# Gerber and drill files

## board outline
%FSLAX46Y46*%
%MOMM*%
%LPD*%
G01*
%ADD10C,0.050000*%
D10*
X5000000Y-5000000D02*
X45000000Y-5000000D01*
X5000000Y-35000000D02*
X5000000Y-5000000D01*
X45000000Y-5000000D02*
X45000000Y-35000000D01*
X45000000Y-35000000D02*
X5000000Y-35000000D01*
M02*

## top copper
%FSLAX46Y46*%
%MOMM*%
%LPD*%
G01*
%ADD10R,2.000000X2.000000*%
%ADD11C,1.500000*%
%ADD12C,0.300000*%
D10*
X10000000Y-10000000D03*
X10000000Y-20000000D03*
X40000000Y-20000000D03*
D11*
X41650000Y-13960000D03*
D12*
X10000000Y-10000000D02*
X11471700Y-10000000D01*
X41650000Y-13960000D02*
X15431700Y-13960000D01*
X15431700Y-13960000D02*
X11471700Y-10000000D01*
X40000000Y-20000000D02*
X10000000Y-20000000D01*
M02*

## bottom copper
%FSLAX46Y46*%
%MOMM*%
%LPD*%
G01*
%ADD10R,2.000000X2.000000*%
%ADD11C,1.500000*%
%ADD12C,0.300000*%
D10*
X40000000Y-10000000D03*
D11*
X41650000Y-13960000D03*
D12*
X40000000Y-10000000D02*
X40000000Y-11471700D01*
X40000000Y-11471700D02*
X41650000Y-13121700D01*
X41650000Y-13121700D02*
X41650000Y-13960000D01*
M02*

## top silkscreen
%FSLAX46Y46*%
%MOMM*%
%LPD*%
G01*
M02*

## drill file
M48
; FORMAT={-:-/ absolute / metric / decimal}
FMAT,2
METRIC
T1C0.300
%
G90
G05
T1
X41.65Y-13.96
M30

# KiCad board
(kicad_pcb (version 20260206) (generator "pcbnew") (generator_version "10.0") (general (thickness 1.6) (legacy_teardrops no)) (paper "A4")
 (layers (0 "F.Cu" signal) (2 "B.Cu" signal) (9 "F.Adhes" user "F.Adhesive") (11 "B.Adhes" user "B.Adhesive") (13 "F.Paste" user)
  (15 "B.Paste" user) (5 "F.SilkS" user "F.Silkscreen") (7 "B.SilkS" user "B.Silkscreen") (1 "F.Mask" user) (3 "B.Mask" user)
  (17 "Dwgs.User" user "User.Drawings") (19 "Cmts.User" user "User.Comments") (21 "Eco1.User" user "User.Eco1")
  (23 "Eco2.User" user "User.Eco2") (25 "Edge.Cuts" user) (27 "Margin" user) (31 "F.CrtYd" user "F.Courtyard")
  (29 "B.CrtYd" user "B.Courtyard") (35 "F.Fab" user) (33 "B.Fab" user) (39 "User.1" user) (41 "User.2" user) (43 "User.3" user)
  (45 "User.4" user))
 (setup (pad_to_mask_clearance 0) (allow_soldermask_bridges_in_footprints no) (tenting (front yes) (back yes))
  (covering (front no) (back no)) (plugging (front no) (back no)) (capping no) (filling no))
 (gr_line (start 5 5) (end 45 5) (stroke (width 0.05) (type default)) (layer "Edge.Cuts"))
 (gr_line (start 5 35) (end 5 5) (stroke (width 0.05) (type default)) (layer "Edge.Cuts"))
 (gr_line (start 45 5) (end 45 35) (stroke (width 0.05) (type default)) (layer "Edge.Cuts"))
 (gr_line (start 45 35) (end 5 35) (stroke (width 0.05) (type default)) (layer "Edge.Cuts"))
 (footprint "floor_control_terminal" (layer "F.Cu") (at 10 10)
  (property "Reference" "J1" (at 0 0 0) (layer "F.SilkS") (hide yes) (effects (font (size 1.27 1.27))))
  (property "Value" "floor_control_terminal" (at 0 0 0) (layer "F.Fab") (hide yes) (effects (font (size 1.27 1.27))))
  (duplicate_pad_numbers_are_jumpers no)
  (pad "1" smd rect (at 0 0) (size 2 2) (layers "F.Cu" "F.Paste" "F.Mask") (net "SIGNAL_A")))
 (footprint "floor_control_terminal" (layer "B.Cu") (at 40 10)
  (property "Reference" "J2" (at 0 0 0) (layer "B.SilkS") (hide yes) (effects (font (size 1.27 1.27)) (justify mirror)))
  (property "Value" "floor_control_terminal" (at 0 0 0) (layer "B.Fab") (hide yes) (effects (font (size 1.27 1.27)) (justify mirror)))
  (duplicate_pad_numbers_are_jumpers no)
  (pad "1" smd rect (at 0 0) (size 2 2) (layers "B.Cu" "B.Paste" "B.Mask") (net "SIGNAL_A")))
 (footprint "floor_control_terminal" (layer "F.Cu") (at 10 20)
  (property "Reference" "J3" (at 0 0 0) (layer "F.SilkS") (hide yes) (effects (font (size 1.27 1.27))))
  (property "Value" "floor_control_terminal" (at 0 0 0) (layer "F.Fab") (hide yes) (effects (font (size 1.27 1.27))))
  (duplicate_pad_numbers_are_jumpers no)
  (pad "1" smd rect (at 0 0) (size 2 2) (layers "F.Cu" "F.Paste" "F.Mask") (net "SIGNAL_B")))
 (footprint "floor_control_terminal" (layer "F.Cu") (at 40 20)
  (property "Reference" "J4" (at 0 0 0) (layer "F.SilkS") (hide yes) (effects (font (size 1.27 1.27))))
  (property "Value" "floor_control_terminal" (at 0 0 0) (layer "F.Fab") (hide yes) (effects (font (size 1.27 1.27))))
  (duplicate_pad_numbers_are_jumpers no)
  (pad "1" smd rect (at 0 0) (size 2 2) (layers "F.Cu" "F.Paste" "F.Mask") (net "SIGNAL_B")))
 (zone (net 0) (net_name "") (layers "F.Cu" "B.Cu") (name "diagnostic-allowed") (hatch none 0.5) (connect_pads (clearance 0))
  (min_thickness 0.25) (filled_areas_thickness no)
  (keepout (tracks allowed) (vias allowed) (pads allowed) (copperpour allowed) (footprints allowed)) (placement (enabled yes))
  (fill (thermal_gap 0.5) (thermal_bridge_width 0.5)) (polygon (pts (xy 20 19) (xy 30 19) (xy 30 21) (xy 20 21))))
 (segment (start 10 10) (end 11.4717 10) (width 0.3) (layer "F.Cu") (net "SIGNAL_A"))
 (segment (start 41.65 13.96) (end 15.4317 13.96) (width 0.3) (layer "F.Cu") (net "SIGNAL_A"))
 (segment (start 15.4317 13.96) (end 11.4717 10) (width 0.3) (layer "F.Cu") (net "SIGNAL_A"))
 (via (at 41.65 13.96) (size 1.5) (drill 0.3) (layers "F.Cu" "B.Cu") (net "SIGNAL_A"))
 (segment (start 40 10) (end 40 11.4717) (width 0.3) (layer "B.Cu") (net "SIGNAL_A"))
 (segment (start 40 11.4717) (end 41.65 13.1217) (width 0.3) (layer "B.Cu") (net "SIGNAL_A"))
 (segment (start 41.65 13.1217) (end 41.65 13.96) (width 0.3) (layer "B.Cu") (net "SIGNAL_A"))
 (segment (start 40 20) (end 10 20) (width 0.3) (layer "F.Cu") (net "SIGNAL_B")))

